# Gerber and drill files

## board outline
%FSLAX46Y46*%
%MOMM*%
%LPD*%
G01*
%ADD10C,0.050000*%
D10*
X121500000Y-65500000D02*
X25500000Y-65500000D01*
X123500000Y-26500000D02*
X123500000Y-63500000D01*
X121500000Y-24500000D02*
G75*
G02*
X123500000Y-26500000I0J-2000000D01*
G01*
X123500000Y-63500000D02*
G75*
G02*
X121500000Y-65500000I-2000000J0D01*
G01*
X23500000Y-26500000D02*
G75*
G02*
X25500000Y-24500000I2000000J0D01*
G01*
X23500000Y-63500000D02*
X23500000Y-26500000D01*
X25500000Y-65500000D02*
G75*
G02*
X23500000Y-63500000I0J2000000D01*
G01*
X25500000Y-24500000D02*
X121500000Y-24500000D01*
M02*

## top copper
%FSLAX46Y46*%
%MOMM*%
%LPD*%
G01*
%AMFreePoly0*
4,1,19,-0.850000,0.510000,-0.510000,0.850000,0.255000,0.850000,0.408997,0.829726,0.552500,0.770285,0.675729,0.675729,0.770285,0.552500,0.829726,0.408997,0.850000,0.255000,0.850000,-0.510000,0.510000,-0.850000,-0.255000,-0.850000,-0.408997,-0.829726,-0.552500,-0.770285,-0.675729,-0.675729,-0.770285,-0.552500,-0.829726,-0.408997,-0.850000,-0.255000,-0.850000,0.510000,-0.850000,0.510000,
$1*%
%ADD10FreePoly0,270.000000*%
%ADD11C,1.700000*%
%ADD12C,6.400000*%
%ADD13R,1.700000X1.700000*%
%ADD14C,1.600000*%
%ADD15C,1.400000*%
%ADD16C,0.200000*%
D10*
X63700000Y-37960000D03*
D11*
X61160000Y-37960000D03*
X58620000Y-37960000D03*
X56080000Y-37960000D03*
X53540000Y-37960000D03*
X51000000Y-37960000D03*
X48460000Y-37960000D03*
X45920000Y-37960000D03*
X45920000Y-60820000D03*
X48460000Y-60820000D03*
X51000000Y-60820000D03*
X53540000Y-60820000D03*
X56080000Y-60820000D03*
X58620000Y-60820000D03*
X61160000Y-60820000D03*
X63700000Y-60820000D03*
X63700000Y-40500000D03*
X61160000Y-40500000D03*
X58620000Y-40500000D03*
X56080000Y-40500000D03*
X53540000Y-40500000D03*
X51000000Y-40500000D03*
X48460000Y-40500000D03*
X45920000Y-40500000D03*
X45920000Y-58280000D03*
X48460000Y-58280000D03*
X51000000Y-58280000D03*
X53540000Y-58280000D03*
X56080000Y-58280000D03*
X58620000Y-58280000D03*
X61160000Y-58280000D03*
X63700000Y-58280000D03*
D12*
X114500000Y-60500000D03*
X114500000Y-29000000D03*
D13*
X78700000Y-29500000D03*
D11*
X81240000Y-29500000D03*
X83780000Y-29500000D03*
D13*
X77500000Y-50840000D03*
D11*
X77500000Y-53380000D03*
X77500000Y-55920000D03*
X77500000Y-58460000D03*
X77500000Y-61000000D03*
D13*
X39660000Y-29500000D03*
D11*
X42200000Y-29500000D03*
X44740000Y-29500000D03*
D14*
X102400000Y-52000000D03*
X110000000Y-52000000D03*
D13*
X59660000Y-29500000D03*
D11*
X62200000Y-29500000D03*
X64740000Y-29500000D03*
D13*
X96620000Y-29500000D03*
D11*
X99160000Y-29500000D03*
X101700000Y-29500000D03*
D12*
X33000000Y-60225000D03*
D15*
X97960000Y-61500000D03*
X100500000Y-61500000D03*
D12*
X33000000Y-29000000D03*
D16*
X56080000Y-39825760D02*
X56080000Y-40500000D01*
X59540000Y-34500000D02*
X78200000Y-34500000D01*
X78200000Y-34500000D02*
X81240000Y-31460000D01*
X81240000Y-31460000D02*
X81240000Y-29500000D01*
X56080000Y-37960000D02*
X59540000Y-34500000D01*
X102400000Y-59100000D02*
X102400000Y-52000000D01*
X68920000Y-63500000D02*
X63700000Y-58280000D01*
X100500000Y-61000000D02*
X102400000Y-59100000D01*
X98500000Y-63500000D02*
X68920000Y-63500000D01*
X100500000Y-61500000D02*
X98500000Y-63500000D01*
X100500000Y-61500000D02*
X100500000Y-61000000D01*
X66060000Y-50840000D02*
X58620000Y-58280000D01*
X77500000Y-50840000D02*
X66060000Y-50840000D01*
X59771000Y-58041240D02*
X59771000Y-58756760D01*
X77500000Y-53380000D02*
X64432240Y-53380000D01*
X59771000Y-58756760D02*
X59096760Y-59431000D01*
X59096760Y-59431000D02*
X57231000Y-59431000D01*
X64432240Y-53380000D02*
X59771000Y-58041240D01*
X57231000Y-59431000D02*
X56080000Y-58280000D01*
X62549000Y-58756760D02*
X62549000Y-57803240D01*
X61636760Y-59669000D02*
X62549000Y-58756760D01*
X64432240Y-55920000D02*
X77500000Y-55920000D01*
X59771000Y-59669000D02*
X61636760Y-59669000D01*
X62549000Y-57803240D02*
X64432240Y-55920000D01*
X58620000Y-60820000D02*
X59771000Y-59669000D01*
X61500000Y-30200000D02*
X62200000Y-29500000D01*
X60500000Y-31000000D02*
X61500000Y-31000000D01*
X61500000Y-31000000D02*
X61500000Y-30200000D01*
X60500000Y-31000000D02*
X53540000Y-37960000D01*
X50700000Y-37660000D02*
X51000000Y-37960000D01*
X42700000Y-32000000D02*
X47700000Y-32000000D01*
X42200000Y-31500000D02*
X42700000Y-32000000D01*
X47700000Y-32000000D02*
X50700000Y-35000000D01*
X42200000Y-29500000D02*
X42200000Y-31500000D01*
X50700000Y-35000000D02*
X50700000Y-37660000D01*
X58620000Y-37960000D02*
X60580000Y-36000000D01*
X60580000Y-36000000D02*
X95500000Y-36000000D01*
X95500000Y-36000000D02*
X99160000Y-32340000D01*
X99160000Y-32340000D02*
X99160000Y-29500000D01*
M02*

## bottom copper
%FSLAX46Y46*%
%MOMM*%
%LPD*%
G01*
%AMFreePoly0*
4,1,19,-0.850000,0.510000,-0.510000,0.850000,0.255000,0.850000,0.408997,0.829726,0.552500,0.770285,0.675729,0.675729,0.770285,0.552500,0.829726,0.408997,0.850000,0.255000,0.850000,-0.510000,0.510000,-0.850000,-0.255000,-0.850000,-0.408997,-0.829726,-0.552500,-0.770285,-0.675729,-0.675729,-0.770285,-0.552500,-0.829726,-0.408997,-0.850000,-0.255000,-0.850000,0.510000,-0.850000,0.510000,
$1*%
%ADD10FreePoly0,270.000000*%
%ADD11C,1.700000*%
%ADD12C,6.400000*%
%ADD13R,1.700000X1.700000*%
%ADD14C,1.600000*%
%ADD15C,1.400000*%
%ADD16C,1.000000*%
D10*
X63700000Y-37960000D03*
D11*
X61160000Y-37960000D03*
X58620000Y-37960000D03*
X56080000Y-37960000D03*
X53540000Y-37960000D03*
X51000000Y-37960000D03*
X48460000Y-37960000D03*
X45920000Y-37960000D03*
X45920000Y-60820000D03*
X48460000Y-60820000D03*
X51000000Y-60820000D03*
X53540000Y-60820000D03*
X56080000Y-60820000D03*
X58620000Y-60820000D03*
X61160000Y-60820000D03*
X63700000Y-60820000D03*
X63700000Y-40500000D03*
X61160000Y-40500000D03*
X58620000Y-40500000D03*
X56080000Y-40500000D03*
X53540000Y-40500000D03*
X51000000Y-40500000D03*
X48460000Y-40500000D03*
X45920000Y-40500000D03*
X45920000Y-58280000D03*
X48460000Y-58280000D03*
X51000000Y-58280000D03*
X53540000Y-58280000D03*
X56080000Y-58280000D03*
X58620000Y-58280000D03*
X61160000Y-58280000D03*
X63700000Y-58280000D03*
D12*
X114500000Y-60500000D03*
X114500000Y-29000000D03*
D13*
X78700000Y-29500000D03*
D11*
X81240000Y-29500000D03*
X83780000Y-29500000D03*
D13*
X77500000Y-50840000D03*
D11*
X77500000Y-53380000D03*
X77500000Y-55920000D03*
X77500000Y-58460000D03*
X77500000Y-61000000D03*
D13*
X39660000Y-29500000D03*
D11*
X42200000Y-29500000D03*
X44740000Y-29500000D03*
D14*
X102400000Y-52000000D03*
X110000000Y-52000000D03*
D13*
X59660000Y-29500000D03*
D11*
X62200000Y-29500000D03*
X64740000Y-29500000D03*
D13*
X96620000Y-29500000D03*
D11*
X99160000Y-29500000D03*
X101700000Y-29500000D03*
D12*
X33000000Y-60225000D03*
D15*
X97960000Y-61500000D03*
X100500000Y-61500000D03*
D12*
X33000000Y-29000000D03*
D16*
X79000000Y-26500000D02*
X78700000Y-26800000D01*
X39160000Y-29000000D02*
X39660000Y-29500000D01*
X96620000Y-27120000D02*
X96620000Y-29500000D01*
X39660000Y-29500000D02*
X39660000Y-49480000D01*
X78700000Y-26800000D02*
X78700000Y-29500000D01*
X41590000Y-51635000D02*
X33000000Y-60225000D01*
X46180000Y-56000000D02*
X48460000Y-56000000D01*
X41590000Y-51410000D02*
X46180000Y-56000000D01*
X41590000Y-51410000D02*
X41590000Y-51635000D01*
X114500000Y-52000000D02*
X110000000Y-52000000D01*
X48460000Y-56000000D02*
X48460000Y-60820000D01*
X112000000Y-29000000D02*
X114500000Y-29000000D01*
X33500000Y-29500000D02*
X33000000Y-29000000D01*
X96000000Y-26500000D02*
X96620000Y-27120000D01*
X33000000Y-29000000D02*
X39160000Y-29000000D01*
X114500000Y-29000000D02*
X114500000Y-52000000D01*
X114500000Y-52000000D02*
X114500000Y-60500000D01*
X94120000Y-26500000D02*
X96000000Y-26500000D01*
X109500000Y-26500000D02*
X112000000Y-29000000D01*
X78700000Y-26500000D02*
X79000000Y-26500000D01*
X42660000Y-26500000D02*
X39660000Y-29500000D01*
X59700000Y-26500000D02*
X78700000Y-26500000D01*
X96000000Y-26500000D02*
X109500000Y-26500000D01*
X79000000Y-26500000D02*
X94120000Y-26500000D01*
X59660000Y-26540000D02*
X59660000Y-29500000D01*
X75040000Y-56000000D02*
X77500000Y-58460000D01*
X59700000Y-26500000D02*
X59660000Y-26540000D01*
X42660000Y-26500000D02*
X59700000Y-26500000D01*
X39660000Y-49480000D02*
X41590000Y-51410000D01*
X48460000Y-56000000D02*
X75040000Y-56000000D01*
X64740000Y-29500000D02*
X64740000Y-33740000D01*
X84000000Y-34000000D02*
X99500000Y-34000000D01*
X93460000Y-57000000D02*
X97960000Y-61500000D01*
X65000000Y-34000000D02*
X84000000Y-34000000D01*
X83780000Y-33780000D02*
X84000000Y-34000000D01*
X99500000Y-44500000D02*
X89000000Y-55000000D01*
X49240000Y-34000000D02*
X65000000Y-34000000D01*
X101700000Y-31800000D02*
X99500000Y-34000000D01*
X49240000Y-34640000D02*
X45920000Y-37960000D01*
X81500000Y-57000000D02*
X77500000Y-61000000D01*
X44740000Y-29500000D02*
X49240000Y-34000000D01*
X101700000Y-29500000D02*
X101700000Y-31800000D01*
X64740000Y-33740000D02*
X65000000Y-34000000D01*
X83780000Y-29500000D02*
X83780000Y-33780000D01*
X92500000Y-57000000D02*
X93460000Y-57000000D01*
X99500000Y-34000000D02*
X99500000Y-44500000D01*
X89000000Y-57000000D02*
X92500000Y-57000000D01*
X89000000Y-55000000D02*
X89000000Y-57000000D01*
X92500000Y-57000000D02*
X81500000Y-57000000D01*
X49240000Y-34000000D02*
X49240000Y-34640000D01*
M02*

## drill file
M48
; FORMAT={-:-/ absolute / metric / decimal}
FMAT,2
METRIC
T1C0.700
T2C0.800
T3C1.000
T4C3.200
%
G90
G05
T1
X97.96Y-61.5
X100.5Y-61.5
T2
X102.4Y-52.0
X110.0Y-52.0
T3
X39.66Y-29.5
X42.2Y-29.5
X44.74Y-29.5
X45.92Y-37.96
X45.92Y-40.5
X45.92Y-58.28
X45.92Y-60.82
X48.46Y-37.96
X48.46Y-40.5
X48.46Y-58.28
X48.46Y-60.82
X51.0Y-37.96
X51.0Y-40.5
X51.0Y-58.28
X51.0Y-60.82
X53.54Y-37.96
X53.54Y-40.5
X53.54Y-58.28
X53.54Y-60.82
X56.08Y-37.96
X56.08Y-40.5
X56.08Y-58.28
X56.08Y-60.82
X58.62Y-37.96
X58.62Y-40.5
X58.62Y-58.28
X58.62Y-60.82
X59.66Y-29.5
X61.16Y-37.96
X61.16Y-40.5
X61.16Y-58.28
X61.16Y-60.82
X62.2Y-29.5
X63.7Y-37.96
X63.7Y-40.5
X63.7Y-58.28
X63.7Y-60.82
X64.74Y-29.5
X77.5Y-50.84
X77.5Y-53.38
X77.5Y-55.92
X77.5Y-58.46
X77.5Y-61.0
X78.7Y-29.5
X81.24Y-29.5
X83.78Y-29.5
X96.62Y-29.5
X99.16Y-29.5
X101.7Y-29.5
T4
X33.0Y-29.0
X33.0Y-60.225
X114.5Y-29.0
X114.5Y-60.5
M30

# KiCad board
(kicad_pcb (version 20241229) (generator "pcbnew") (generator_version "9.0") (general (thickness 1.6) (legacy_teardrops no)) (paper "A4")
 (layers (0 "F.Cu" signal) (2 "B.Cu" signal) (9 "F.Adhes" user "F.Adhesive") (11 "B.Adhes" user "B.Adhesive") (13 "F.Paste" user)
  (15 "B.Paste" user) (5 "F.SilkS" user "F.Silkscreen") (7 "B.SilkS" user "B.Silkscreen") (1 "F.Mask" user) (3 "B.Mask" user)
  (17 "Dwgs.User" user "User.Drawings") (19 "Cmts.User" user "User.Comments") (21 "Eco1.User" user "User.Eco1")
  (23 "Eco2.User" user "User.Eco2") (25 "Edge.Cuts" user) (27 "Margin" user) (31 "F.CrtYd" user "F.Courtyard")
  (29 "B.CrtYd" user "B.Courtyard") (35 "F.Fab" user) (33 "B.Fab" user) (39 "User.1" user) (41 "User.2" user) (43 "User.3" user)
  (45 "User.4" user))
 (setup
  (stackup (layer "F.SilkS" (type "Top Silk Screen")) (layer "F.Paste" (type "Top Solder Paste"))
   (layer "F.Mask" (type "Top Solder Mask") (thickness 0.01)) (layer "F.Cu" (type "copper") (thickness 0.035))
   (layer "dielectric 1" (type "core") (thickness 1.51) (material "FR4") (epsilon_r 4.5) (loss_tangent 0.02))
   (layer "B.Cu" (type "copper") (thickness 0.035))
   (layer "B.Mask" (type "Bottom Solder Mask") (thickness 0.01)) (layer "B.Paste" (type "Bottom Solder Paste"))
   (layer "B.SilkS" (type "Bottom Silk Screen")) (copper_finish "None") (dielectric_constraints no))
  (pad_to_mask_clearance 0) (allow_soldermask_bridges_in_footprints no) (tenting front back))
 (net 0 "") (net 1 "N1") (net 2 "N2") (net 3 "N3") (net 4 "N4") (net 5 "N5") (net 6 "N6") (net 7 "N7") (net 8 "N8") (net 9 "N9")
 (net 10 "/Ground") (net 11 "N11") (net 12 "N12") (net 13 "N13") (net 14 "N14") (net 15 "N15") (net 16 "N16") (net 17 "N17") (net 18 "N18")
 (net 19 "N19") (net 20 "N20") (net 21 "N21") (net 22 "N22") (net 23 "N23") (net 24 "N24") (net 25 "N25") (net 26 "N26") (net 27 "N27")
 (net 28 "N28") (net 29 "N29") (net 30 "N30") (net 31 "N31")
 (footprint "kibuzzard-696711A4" (layer "F.Cu") (at 95.5 41)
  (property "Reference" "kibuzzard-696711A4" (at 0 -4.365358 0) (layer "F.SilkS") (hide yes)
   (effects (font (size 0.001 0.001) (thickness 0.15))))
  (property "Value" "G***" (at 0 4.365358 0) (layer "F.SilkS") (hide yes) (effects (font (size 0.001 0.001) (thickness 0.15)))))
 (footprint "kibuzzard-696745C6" (layer "F.Cu") (at 95.5 44.5)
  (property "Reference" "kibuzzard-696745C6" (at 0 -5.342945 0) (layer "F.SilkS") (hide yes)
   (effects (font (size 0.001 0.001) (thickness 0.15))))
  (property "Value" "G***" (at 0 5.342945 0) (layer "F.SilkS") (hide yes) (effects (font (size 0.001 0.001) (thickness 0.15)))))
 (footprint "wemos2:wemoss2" (layer "F.Cu") (at 63.7 37.96 -90)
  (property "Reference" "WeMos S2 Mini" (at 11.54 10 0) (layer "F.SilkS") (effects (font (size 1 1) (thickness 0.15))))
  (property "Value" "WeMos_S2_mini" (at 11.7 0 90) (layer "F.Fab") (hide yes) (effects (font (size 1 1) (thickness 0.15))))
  (pad "1" thru_hole roundrect (at 0 0 270) (size 1.7 1.7) (drill 1) (layers "*.Cu" "*.Mask") (remove_unused_layers no)
   (roundrect_rratio 0.35) (chamfer_ratio 0.2) (chamfer top_left bottom_right) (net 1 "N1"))
  (pad "2" thru_hole circle (at 0 2.54 270) (size 1.7 1.7) (drill 1) (layers "*.Cu" "*.Mask") (remove_unused_layers no) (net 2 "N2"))
  (pad "3" thru_hole circle (at 0 5.08 270) (size 1.7 1.7) (drill 1) (layers "*.Cu" "*.Mask") (remove_unused_layers no) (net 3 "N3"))
  (pad "4" thru_hole circle (at 0 7.62 270) (size 1.7 1.7) (drill 1) (layers "*.Cu" "*.Mask") (remove_unused_layers no) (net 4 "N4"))
  (pad "5" thru_hole circle (at 0 10.16 270) (size 1.7 1.7) (drill 1) (layers "*.Cu" "*.Mask") (remove_unused_layers no) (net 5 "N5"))
  (pad "6" thru_hole circle (at 0 12.7 270) (size 1.7 1.7) (drill 1) (layers "*.Cu" "*.Mask") (remove_unused_layers no) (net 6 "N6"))
  (pad "7" thru_hole circle (at 0 15.24 270) (size 1.7 1.7) (drill 1) (layers "*.Cu" "*.Mask") (remove_unused_layers no) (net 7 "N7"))
  (pad "8" thru_hole circle (at 0 17.78 270) (size 1.7 1.7) (drill 1) (layers "*.Cu" "*.Mask") (remove_unused_layers no) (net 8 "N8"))
  (pad "9" thru_hole circle (at 22.86 17.78 270) (size 1.7 1.7) (drill 1) (layers "*.Cu" "*.Mask") (remove_unused_layers no) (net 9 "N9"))
  (pad "10" thru_hole circle (at 22.86 15.24 270) (size 1.7 1.7) (drill 1) (layers "*.Cu" "*.Mask") (remove_unused_layers no)
   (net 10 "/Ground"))
  (pad "11" thru_hole circle (at 22.86 12.7 270) (size 1.7 1.7) (drill 1) (layers "*.Cu" "*.Mask") (remove_unused_layers no) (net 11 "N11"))
  (pad "12" thru_hole circle (at 22.86 10.16 270) (size 1.7 1.7) (drill 1) (layers "*.Cu" "*.Mask") (remove_unused_layers no) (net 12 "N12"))
  (pad "13" thru_hole circle (at 22.86 7.62 270) (size 1.7 1.7) (drill 1) (layers "*.Cu" "*.Mask") (remove_unused_layers no) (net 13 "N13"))
  (pad "14" thru_hole circle (at 22.86 5.08 270) (size 1.7 1.7) (drill 1) (layers "*.Cu" "*.Mask") (remove_unused_layers no) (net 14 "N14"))
  (pad "15" thru_hole circle (at 22.86 2.54 270) (size 1.7 1.7) (drill 1) (layers "*.Cu" "*.Mask") (remove_unused_layers no) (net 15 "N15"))
  (pad "16" thru_hole circle (at 22.86 0 270) (size 1.7 1.7) (drill 1) (layers "*.Cu" "*.Mask") (remove_unused_layers no) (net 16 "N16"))
  (pad "17" thru_hole circle (at 2.54 0 270) (size 1.7 1.7) (drill 1) (layers "*.Cu" "*.Mask") (remove_unused_layers no) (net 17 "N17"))
  (pad "18" thru_hole circle (at 2.54 2.54 270) (size 1.7 1.7) (drill 1) (layers "*.Cu" "*.Mask") (remove_unused_layers no) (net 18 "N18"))
  (pad "19" thru_hole circle (at 2.54 5.08 270) (size 1.7 1.7) (drill 1) (layers "*.Cu" "*.Mask") (remove_unused_layers no) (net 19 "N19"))
  (pad "20" thru_hole circle (at 2.54 7.62 270) (size 1.7 1.7) (drill 1) (layers "*.Cu" "*.Mask") (remove_unused_layers no) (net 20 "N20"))
  (pad "21" thru_hole circle (at 2.54 10.16 270) (size 1.7 1.7) (drill 1) (layers "*.Cu" "*.Mask") (remove_unused_layers no) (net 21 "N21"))
  (pad "22" thru_hole circle (at 2.54 12.7 270) (size 1.7 1.7) (drill 1) (layers "*.Cu" "*.Mask") (remove_unused_layers no) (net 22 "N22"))
  (pad "23" thru_hole circle (at 2.54 15.24 270) (size 1.7 1.7) (drill 1) (layers "*.Cu" "*.Mask") (remove_unused_layers no) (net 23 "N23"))
  (pad "24" thru_hole circle (at 2.54 17.78 270) (size 1.7 1.7) (drill 1) (layers "*.Cu" "*.Mask") (remove_unused_layers no) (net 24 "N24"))
  (pad "25" thru_hole circle (at 20.32 17.78 270) (size 1.7 1.7) (drill 1) (layers "*.Cu" "*.Mask") (remove_unused_layers no) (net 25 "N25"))
  (pad "26" thru_hole circle (at 20.32 15.24 270) (size 1.7 1.7) (drill 1) (layers "*.Cu" "*.Mask") (remove_unused_layers no)
   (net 10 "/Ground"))
  (pad "27" thru_hole circle (at 20.32 12.7 270) (size 1.7 1.7) (drill 1) (layers "*.Cu" "*.Mask") (remove_unused_layers no) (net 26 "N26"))
  (pad "28" thru_hole circle (at 20.32 10.16 270) (size 1.7 1.7) (drill 1) (layers "*.Cu" "*.Mask") (remove_unused_layers no) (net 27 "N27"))
  (pad "29" thru_hole circle (at 20.32 7.62 270) (size 1.7 1.7) (drill 1) (layers "*.Cu" "*.Mask") (remove_unused_layers no) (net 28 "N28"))
  (pad "30" thru_hole circle (at 20.32 5.08 270) (size 1.7 1.7) (drill 1) (layers "*.Cu" "*.Mask") (remove_unused_layers no) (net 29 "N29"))
  (pad "31" thru_hole circle (at 20.32 2.54 270) (size 1.7 1.7) (drill 1) (layers "*.Cu" "*.Mask") (remove_unused_layers no) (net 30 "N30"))
  (pad "32" thru_hole circle (at 20.32 0 270) (size 1.7 1.7) (drill 1) (layers "*.Cu" "*.Mask") (remove_unused_layers no) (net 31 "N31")))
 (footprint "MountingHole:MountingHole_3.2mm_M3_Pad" (layer "F.Cu") (at 114.5 60.5)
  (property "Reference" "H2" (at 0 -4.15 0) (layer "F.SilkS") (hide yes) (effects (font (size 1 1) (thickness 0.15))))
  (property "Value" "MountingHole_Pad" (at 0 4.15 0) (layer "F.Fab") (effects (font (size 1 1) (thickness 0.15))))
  (pad "1" thru_hole circle (at 0 0) (size 6.4 6.4) (drill 3.2) (layers "*.Cu" "*.Mask") (remove_unused_layers no) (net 10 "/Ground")
   (zone_connect 2)))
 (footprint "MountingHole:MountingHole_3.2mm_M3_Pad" (layer "F.Cu") (at 114.5 29)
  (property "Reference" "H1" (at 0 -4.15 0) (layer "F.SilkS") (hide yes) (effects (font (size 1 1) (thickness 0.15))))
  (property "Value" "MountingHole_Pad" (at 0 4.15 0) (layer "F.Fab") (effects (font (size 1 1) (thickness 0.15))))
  (pad "1" thru_hole circle (at 0 0) (size 6.4 6.4) (drill 3.2) (layers "*.Cu" "*.Mask") (remove_unused_layers no) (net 10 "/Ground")
   (zone_connect 2)))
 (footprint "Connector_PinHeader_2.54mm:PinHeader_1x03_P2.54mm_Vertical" (layer "F.Cu") (at 78.7 29.5 90)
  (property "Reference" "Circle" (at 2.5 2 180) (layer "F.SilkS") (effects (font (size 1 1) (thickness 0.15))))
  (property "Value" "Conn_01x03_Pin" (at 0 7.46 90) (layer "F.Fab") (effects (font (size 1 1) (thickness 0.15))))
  (pad "1" thru_hole rect (at 0 0 90) (size 1.7 1.7) (drill 1) (layers "*.Cu" "*.Mask") (remove_unused_layers no) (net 10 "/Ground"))
  (pad "2" thru_hole circle (at 0 2.54 90) (size 1.7 1.7) (drill 1) (layers "*.Cu" "*.Mask") (remove_unused_layers no) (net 4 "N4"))
  (pad "3" thru_hole circle (at 0 5.08 90) (size 1.7 1.7) (drill 1) (layers "*.Cu" "*.Mask") (remove_unused_layers no) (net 8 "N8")))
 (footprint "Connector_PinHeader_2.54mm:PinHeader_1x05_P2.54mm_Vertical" (layer "F.Cu") (at 77.5 50.84)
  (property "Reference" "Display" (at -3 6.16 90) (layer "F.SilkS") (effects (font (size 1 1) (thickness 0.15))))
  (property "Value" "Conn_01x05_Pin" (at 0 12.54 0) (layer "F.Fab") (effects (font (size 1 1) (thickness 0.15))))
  (pad "1" thru_hole rect (at 0 0) (size 1.7 1.7) (drill 1) (layers "*.Cu" "*.Mask") (remove_unused_layers no) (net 29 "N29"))
  (pad "2" thru_hole circle (at 0 2.54) (size 1.7 1.7) (drill 1) (layers "*.Cu" "*.Mask") (remove_unused_layers no) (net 28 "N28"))
  (pad "3" thru_hole circle (at 0 5.08) (size 1.7 1.7) (drill 1) (layers "*.Cu" "*.Mask") (remove_unused_layers no) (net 14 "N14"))
  (pad "4" thru_hole circle (at 0 7.62) (size 1.7 1.7) (drill 1) (layers "*.Cu" "*.Mask") (remove_unused_layers no) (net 10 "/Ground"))
  (pad "5" thru_hole circle (at 0 10.16) (size 1.7 1.7) (drill 1) (layers "*.Cu" "*.Mask") (remove_unused_layers no) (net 8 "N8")))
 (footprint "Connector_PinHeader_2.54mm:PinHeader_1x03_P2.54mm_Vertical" (layer "F.Cu") (at 39.66 29.5 90)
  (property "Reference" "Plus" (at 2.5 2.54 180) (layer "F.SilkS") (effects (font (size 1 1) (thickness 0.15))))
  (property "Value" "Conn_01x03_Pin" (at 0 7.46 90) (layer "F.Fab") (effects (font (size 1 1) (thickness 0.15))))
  (pad "1" thru_hole rect (at 0 0 90) (size 1.7 1.7) (drill 1) (layers "*.Cu" "*.Mask") (remove_unused_layers no) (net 10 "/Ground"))
  (pad "2" thru_hole circle (at 0 2.54 90) (size 1.7 1.7) (drill 1) (layers "*.Cu" "*.Mask") (remove_unused_layers no) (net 6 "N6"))
  (pad "3" thru_hole circle (at 0 5.08 90) (size 1.7 1.7) (drill 1) (layers "*.Cu" "*.Mask") (remove_unused_layers no) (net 8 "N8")))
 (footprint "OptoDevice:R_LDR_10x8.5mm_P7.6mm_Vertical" (layer "F.Cu") (at 102.4 52)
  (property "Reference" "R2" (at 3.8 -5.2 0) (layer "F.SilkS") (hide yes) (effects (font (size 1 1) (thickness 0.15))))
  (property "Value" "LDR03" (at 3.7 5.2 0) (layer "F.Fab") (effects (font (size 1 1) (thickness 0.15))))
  (pad "1" thru_hole circle (at 0 0) (size 1.6 1.6) (drill 0.8) (layers "*.Cu" "*.Mask") (remove_unused_layers no) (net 31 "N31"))
  (pad "2" thru_hole circle (at 7.6 0) (size 1.6 1.6) (drill 0.8) (layers "*.Cu" "*.Mask") (remove_unused_layers no) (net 10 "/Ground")))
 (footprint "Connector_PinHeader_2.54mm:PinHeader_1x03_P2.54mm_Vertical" (layer "F.Cu") (at 59.66 29.5 90)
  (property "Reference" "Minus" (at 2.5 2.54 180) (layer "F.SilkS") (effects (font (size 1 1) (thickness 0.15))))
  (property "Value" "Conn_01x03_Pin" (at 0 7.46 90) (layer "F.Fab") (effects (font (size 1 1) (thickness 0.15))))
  (pad "1" thru_hole rect (at 0 0 90) (size 1.7 1.7) (drill 1) (layers "*.Cu" "*.Mask") (remove_unused_layers no) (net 10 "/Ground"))
  (pad "2" thru_hole circle (at 0 2.54 90) (size 1.7 1.7) (drill 1) (layers "*.Cu" "*.Mask") (remove_unused_layers no) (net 5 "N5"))
  (pad "3" thru_hole circle (at 0 5.08 90) (size 1.7 1.7) (drill 1) (layers "*.Cu" "*.Mask") (remove_unused_layers no) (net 8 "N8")))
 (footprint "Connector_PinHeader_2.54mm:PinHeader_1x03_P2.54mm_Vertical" (layer "F.Cu") (at 96.62 29.5 90)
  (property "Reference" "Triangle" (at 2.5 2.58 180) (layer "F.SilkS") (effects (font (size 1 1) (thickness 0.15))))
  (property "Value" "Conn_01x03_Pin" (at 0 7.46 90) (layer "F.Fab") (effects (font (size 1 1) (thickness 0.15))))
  (pad "1" thru_hole rect (at 0 0 90) (size 1.7 1.7) (drill 1) (layers "*.Cu" "*.Mask") (remove_unused_layers no) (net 10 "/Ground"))
  (pad "2" thru_hole circle (at 0 2.54 90) (size 1.7 1.7) (drill 1) (layers "*.Cu" "*.Mask") (remove_unused_layers no) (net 3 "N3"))
  (pad "3" thru_hole circle (at 0 5.08 90) (size 1.7 1.7) (drill 1) (layers "*.Cu" "*.Mask") (remove_unused_layers no) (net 8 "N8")))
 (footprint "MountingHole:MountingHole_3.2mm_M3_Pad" (layer "F.Cu") (at 33 60.225)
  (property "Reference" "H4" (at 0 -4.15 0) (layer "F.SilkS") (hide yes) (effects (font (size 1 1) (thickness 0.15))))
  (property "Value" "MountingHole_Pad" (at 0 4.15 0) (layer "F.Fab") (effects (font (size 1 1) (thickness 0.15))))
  (pad "1" thru_hole circle (at 0 0) (size 6.4 6.4) (drill 3.2) (layers "*.Cu" "*.Mask") (remove_unused_layers no) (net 10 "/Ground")
   (zone_connect 2)))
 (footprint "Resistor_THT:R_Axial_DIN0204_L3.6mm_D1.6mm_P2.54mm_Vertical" (layer "F.Cu") (at 97.96 61.5)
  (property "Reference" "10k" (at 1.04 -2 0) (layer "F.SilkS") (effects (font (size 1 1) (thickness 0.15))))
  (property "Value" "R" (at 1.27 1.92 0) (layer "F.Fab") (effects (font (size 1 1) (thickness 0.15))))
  (pad "1" thru_hole circle (at 0 0) (size 1.4 1.4) (drill 0.7) (layers "*.Cu" "*.Mask") (remove_unused_layers no) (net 8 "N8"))
  (pad "2" thru_hole circle (at 2.54 0) (size 1.4 1.4) (drill 0.7) (layers "*.Cu" "*.Mask") (remove_unused_layers no) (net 31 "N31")))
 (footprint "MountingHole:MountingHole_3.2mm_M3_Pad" (layer "F.Cu") (at 33 29)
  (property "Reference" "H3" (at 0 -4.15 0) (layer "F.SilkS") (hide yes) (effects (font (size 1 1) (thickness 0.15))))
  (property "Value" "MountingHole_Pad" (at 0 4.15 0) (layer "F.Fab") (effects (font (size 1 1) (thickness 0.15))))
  (pad "1" thru_hole circle (at 0 0) (size 6.4 6.4) (drill 3.2) (layers "*.Cu" "*.Mask") (remove_unused_layers no) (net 10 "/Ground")
   (zone_connect 2)))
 (gr_line (start 121.5 65.5) (end 25.5 65.5) (stroke (width 0.05) (type default)) (layer "Edge.Cuts"))
 (gr_line (start 123.5 26.5) (end 123.5 63.5) (stroke (width 0.05) (type default)) (layer "Edge.Cuts"))
 (gr_arc (start 121.5 24.5) (mid 122.914214 25.085786) (end 123.5 26.5) (stroke (width 0.05) (type default)) (layer "Edge.Cuts"))
 (gr_arc (start 123.5 63.5) (mid 122.914214 64.914214) (end 121.5 65.5) (stroke (width 0.05) (type default)) (layer "Edge.Cuts"))
 (gr_arc (start 23.5 26.5) (mid 24.085786 25.085786) (end 25.5 24.5) (stroke (width 0.05) (type default)) (layer "Edge.Cuts"))
 (gr_line (start 23.5 63.5) (end 23.5 26.5) (stroke (width 0.05) (type default)) (layer "Edge.Cuts"))
 (gr_arc (start 25.5 65.5) (mid 24.085786 64.914214) (end 23.5 63.5) (stroke (width 0.05) (type default)) (layer "Edge.Cuts"))
 (gr_line (start 25.5 24.5) (end 121.5 24.5) (stroke (width 0.05) (type default)) (layer "Edge.Cuts"))
 (segment (start 79 26.5) (end 78.7 26.8) (width 1) (layer "B.Cu") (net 10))
 (segment (start 39.16 29) (end 39.66 29.5) (width 1) (layer "B.Cu") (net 10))
 (segment (start 96.62 27.12) (end 96.62 29.5) (width 1) (layer "B.Cu") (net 10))
 (segment (start 39.66 29.5) (end 39.66 49.48) (width 1) (layer "B.Cu") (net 10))
 (segment (start 78.7 26.8) (end 78.7 29.5) (width 1) (layer "B.Cu") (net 10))
 (segment (start 41.59 51.635) (end 33 60.225) (width 1) (layer "B.Cu") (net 10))
 (segment (start 46.18 56) (end 48.46 56) (width 1) (layer "B.Cu") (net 10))
 (segment (start 41.59 51.41) (end 46.18 56) (width 1) (layer "B.Cu") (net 10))
 (segment (start 41.59 51.41) (end 41.59 51.635) (width 1) (layer "B.Cu") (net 10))
 (segment (start 114.5 52) (end 110 52) (width 1) (layer "B.Cu") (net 10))
 (segment (start 48.46 56) (end 48.46 60.82) (width 1) (layer "B.Cu") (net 10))
 (segment (start 112 29) (end 114.5 29) (width 1) (layer "B.Cu") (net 10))
 (segment (start 33.5 29.5) (end 33 29) (width 1) (layer "B.Cu") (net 10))
 (segment (start 96 26.5) (end 96.62 27.12) (width 1) (layer "B.Cu") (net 10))
 (segment (start 33 29) (end 39.16 29) (width 1) (layer "B.Cu") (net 10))
 (segment (start 114.5 29) (end 114.5 52) (width 1) (layer "B.Cu") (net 10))
 (segment (start 114.5 52) (end 114.5 60.5) (width 1) (layer "B.Cu") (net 10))
 (segment (start 94.12 26.5) (end 96 26.5) (width 1) (layer "B.Cu") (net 10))
 (segment (start 109.5 26.5) (end 112 29) (width 1) (layer "B.Cu") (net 10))
 (segment (start 78.7 26.5) (end 79 26.5) (width 1) (layer "B.Cu") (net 10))
 (segment (start 42.66 26.5) (end 39.66 29.5) (width 1) (layer "B.Cu") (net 10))
 (segment (start 59.7 26.5) (end 78.7 26.5) (width 1) (layer "B.Cu") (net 10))
 (segment (start 96 26.5) (end 109.5 26.5) (width 1) (layer "B.Cu") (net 10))
 (segment (start 79 26.5) (end 94.12 26.5) (width 1) (layer "B.Cu") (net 10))
 (segment (start 59.66 26.54) (end 59.66 29.5) (width 1) (layer "B.Cu") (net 10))
 (segment (start 75.04 56) (end 77.5 58.46) (width 1) (layer "B.Cu") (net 10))
 (segment (start 59.7 26.5) (end 59.66 26.54) (width 1) (layer "B.Cu") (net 10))
 (segment (start 42.66 26.5) (end 59.7 26.5) (width 1) (layer "B.Cu") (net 10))
 (segment (start 39.66 49.48) (end 41.59 51.41) (width 1) (layer "B.Cu") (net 10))
 (segment (start 48.46 56) (end 75.04 56) (width 1) (layer "B.Cu") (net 10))
 (segment (start 56.08 39.82576) (end 56.08 40.5) (width 0.2) (layer "F.Cu") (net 20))
 (segment (start 64.74 29.5) (end 64.74 33.74) (width 1) (layer "B.Cu") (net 8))
 (segment (start 84 34) (end 99.5 34) (width 1) (layer "B.Cu") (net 8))
 (segment (start 93.46 57) (end 97.96 61.5) (width 1) (layer "B.Cu") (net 8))
 (segment (start 65 34) (end 84 34) (width 1) (layer "B.Cu") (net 8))
 (segment (start 83.78 33.78) (end 84 34) (width 1) (layer "B.Cu") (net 8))
 (segment (start 99.5 44.5) (end 89 55) (width 1) (layer "B.Cu") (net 8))
 (segment (start 49.24 34) (end 65 34) (width 1) (layer "B.Cu") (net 8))
 (segment (start 101.7 31.8) (end 99.5 34) (width 1) (layer "B.Cu") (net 8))
 (segment (start 49.24 34.64) (end 45.92 37.96) (width 1) (layer "B.Cu") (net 8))
 (segment (start 81.5 57) (end 77.5 61) (width 1) (layer "B.Cu") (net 8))
 (segment (start 44.74 29.5) (end 49.24 34) (width 1) (layer "B.Cu") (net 8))
 (segment (start 101.7 29.5) (end 101.7 31.8) (width 1) (layer "B.Cu") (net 8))
 (segment (start 64.74 33.74) (end 65 34) (width 1) (layer "B.Cu") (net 8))
 (segment (start 83.78 29.5) (end 83.78 33.78) (width 1) (layer "B.Cu") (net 8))
 (segment (start 92.5 57) (end 93.46 57) (width 1) (layer "B.Cu") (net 8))
 (segment (start 99.5 34) (end 99.5 44.5) (width 1) (layer "B.Cu") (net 8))
 (segment (start 89 57) (end 92.5 57) (width 1) (layer "B.Cu") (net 8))
 (segment (start 89 55) (end 89 57) (width 1) (layer "B.Cu") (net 8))
 (segment (start 92.5 57) (end 81.5 57) (width 1) (layer "B.Cu") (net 8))
 (segment (start 49.24 34) (end 49.24 34.64) (width 1) (layer "B.Cu") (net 8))
 (segment (start 59.54 34.5) (end 78.2 34.5) (width 0.2) (layer "F.Cu") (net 4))
 (segment (start 78.2 34.5) (end 81.24 31.46) (width 0.2) (layer "F.Cu") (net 4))
 (segment (start 81.24 31.46) (end 81.24 29.5) (width 0.2) (layer "F.Cu") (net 4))
 (segment (start 56.08 37.96) (end 59.54 34.5) (width 0.2) (layer "F.Cu") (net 4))
 (segment (start 102.4 59.1) (end 102.4 52) (width 0.2) (layer "F.Cu") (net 31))
 (segment (start 68.92 63.5) (end 63.7 58.28) (width 0.2) (layer "F.Cu") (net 31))
 (segment (start 100.5 61) (end 102.4 59.1) (width 0.2) (layer "F.Cu") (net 31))
 (segment (start 98.5 63.5) (end 68.92 63.5) (width 0.2) (layer "F.Cu") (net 31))
 (segment (start 100.5 61.5) (end 98.5 63.5) (width 0.2) (layer "F.Cu") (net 31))
 (segment (start 100.5 61.5) (end 100.5 61) (width 0.2) (layer "F.Cu") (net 31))
 (segment (start 66.06 50.84) (end 58.62 58.28) (width 0.2) (layer "F.Cu") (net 29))
 (segment (start 77.5 50.84) (end 66.06 50.84) (width 0.2) (layer "F.Cu") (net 29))
 (segment (start 59.771 58.04124) (end 59.771 58.75676) (width 0.2) (layer "F.Cu") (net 28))
 (segment (start 77.5 53.38) (end 64.43224 53.38) (width 0.2) (layer "F.Cu") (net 28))
 (segment (start 59.771 58.75676) (end 59.09676 59.431) (width 0.2) (layer "F.Cu") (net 28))
 (segment (start 59.09676 59.431) (end 57.231 59.431) (width 0.2) (layer "F.Cu") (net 28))
 (segment (start 64.43224 53.38) (end 59.771 58.04124) (width 0.2) (layer "F.Cu") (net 28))
 (segment (start 57.231 59.431) (end 56.08 58.28) (width 0.2) (layer "F.Cu") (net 28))
 (segment (start 62.549 58.75676) (end 62.549 57.80324) (width 0.2) (layer "F.Cu") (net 14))
 (segment (start 61.63676 59.669) (end 62.549 58.75676) (width 0.2) (layer "F.Cu") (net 14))
 (segment (start 64.43224 55.92) (end 77.5 55.92) (width 0.2) (layer "F.Cu") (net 14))
 (segment (start 59.771 59.669) (end 61.63676 59.669) (width 0.2) (layer "F.Cu") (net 14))
 (segment (start 62.549 57.80324) (end 64.43224 55.92) (width 0.2) (layer "F.Cu") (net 14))
 (segment (start 58.62 60.82) (end 59.771 59.669) (width 0.2) (layer "F.Cu") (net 14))
 (segment (start 61.5 30.2) (end 62.2 29.5) (width 0.2) (layer "F.Cu") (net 5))
 (segment (start 60.5 31) (end 61.5 31) (width 0.2) (layer "F.Cu") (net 5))
 (segment (start 61.5 31) (end 61.5 30.2) (width 0.2) (layer "F.Cu") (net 5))
 (segment (start 60.5 31) (end 53.54 37.96) (width 0.2) (layer "F.Cu") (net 5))
 (segment (start 50.7 37.66) (end 51 37.96) (width 0.2) (layer "F.Cu") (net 6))
 (segment (start 42.7 32) (end 47.7 32) (width 0.2) (layer "F.Cu") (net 6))
 (segment (start 42.2 31.5) (end 42.7 32) (width 0.2) (layer "F.Cu") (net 6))
 (segment (start 47.7 32) (end 50.7 35) (width 0.2) (layer "F.Cu") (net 6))
 (segment (start 42.2 29.5) (end 42.2 31.5) (width 0.2) (layer "F.Cu") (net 6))
 (segment (start 50.7 35) (end 50.7 37.66) (width 0.2) (layer "F.Cu") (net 6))
 (segment (start 58.62 37.96) (end 60.58 36) (width 0.2) (layer "F.Cu") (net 3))
 (segment (start 60.58 36) (end 95.5 36) (width 0.2) (layer "F.Cu") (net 3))
 (segment (start 95.5 36) (end 99.16 32.34) (width 0.2) (layer "F.Cu") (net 3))
 (segment (start 99.16 32.34) (end 99.16 29.5) (width 0.2) (layer "F.Cu") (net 3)))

